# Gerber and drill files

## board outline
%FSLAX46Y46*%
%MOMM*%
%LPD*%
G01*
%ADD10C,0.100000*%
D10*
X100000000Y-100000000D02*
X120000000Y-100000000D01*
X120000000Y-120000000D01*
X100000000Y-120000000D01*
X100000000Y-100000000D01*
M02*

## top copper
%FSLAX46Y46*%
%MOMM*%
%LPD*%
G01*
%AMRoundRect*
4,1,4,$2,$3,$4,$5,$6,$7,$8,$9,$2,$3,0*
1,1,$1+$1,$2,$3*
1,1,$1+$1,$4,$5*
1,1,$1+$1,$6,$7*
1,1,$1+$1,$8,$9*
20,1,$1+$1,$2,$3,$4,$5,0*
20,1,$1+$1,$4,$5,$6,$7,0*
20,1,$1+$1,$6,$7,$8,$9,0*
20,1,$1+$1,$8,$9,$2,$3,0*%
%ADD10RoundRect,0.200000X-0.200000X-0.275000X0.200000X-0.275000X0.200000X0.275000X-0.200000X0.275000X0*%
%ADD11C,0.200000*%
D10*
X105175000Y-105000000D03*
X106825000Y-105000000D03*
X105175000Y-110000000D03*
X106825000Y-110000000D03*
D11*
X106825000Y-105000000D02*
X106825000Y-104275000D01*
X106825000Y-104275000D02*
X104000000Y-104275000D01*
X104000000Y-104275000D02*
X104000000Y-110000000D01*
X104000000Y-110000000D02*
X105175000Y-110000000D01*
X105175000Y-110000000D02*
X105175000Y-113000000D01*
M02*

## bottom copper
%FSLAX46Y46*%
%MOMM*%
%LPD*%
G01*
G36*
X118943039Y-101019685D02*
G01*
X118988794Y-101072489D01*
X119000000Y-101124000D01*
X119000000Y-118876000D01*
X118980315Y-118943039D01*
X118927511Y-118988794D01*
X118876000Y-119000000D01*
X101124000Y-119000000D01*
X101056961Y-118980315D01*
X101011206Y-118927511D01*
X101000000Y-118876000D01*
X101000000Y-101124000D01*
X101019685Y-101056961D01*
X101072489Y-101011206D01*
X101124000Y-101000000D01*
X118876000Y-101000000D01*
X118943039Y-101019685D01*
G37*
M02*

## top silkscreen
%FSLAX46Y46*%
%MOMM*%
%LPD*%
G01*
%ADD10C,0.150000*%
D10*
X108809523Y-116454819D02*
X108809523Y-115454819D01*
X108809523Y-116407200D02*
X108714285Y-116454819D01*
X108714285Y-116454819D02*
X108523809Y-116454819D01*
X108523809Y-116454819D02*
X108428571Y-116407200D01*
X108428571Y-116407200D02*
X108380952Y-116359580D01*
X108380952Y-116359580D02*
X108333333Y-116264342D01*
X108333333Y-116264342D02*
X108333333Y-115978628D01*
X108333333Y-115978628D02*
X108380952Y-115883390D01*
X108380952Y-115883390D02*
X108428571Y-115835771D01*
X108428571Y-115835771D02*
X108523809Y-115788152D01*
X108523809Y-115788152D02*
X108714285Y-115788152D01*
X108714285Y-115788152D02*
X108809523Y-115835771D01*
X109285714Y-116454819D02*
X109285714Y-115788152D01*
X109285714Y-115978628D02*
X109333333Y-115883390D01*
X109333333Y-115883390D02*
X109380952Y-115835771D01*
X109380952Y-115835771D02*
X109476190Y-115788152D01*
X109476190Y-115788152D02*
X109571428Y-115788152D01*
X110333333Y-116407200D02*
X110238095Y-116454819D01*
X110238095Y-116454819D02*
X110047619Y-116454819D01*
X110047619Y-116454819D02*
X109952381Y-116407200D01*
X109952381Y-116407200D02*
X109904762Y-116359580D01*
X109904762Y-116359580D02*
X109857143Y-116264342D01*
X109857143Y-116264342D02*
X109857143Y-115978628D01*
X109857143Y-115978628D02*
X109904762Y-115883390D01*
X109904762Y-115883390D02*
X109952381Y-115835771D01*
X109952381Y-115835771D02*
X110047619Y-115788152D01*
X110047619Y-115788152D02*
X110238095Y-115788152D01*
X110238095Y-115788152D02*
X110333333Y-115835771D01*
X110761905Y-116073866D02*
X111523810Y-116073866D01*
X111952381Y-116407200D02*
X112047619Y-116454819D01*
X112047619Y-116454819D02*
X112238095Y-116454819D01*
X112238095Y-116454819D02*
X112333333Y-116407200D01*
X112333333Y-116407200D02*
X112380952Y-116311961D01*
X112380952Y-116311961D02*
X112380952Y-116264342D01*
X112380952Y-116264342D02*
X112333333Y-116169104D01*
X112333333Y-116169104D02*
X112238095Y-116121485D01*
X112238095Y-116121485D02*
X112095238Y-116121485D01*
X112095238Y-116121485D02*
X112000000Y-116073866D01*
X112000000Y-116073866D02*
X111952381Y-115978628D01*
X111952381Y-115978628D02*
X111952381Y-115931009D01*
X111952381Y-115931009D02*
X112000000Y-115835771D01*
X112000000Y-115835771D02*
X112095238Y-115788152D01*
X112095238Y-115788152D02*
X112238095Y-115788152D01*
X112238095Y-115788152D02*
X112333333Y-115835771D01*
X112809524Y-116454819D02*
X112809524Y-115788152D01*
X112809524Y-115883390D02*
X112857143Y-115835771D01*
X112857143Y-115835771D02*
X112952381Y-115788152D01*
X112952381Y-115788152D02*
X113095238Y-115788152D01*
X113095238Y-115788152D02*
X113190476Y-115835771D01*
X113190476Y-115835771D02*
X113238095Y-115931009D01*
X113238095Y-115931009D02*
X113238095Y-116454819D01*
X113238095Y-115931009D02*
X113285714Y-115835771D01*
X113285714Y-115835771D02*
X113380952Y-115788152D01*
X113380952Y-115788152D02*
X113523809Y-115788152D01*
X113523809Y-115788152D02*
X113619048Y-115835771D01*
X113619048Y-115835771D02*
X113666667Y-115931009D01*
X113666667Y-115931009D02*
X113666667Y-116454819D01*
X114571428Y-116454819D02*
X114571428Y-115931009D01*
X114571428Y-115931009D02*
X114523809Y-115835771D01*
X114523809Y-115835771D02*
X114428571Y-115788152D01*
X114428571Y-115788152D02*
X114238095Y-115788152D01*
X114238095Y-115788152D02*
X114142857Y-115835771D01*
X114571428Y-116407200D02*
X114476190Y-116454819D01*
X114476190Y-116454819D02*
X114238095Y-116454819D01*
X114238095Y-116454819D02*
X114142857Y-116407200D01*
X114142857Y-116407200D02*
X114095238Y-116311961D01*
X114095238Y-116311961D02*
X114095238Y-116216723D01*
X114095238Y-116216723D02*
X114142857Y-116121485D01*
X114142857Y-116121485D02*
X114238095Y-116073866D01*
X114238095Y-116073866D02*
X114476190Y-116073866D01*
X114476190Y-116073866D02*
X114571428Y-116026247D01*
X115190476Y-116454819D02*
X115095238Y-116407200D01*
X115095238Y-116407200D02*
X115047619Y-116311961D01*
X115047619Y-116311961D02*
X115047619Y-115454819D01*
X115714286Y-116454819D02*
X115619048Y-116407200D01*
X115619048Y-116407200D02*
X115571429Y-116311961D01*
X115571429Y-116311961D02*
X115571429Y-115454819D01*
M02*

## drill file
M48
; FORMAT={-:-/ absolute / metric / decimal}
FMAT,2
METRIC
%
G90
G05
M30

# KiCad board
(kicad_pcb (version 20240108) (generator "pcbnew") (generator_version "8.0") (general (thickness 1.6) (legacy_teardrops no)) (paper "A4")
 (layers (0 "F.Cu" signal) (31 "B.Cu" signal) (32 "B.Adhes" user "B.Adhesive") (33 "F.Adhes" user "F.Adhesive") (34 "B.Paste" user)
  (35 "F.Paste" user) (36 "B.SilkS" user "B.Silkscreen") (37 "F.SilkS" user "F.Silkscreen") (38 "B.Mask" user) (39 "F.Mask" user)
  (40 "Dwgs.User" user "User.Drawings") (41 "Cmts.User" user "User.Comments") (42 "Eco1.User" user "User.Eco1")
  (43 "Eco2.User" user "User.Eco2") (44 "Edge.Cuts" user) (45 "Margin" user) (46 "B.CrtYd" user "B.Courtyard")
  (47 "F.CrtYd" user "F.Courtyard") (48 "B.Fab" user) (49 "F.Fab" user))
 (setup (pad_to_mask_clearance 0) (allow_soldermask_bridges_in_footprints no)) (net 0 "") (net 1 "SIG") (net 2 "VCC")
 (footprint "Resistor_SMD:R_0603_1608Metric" (layer "F.Cu") (at 106 105)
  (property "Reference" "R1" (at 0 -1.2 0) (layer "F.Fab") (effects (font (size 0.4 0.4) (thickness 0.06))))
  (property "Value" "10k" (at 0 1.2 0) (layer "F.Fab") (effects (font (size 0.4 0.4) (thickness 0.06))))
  (pad "1" smd roundrect (at -0.825 0) (size 0.8 0.95) (layers "F.Cu" "F.Mask" "F.Paste") (roundrect_rratio 0.25) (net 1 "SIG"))
  (pad "2" smd roundrect (at 0.825 0) (size 0.8 0.95) (layers "F.Cu" "F.Mask" "F.Paste") (roundrect_rratio 0.25) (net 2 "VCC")))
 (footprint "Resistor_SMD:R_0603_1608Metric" (layer "F.Cu") (at 106 110)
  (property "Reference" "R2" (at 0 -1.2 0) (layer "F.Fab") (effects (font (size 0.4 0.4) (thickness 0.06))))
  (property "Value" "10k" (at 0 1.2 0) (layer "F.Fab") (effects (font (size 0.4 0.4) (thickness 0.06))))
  (pad "1" smd roundrect (at -0.825 0) (size 0.8 0.95) (layers "F.Cu" "F.Mask" "F.Paste") (roundrect_rratio 0.25) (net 2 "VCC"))
  (pad "2" smd roundrect (at 0.825 0) (size 0.8 0.95) (layers "F.Cu" "F.Mask" "F.Paste") (roundrect_rratio 0.25) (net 1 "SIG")))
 (segment (start 106.825 105) (end 106.825 104.275) (width 0.2) (layer "F.Cu") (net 2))
 (segment (start 106.825 104.275) (end 104 104.275) (width 0.2) (layer "F.Cu") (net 2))
 (segment (start 104 104.275) (end 104 110) (width 0.2) (layer "F.Cu") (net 2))
 (segment (start 104 110) (end 105.175 110) (width 0.2) (layer "F.Cu") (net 2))
 (segment (start 105.175 110) (end 105.175 113) (width 0.2) (layer "F.Cu") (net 2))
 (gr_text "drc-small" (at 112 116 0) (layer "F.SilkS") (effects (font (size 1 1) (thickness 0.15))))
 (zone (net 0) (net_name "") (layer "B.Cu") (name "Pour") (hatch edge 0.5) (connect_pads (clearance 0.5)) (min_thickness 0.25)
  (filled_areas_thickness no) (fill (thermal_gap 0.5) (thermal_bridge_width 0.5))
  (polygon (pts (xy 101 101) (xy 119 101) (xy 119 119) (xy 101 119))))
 (gr_rect (start 100 100) (end 120 120) (stroke (width 0.1) (type default)) (fill none) (layer "Edge.Cuts")))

